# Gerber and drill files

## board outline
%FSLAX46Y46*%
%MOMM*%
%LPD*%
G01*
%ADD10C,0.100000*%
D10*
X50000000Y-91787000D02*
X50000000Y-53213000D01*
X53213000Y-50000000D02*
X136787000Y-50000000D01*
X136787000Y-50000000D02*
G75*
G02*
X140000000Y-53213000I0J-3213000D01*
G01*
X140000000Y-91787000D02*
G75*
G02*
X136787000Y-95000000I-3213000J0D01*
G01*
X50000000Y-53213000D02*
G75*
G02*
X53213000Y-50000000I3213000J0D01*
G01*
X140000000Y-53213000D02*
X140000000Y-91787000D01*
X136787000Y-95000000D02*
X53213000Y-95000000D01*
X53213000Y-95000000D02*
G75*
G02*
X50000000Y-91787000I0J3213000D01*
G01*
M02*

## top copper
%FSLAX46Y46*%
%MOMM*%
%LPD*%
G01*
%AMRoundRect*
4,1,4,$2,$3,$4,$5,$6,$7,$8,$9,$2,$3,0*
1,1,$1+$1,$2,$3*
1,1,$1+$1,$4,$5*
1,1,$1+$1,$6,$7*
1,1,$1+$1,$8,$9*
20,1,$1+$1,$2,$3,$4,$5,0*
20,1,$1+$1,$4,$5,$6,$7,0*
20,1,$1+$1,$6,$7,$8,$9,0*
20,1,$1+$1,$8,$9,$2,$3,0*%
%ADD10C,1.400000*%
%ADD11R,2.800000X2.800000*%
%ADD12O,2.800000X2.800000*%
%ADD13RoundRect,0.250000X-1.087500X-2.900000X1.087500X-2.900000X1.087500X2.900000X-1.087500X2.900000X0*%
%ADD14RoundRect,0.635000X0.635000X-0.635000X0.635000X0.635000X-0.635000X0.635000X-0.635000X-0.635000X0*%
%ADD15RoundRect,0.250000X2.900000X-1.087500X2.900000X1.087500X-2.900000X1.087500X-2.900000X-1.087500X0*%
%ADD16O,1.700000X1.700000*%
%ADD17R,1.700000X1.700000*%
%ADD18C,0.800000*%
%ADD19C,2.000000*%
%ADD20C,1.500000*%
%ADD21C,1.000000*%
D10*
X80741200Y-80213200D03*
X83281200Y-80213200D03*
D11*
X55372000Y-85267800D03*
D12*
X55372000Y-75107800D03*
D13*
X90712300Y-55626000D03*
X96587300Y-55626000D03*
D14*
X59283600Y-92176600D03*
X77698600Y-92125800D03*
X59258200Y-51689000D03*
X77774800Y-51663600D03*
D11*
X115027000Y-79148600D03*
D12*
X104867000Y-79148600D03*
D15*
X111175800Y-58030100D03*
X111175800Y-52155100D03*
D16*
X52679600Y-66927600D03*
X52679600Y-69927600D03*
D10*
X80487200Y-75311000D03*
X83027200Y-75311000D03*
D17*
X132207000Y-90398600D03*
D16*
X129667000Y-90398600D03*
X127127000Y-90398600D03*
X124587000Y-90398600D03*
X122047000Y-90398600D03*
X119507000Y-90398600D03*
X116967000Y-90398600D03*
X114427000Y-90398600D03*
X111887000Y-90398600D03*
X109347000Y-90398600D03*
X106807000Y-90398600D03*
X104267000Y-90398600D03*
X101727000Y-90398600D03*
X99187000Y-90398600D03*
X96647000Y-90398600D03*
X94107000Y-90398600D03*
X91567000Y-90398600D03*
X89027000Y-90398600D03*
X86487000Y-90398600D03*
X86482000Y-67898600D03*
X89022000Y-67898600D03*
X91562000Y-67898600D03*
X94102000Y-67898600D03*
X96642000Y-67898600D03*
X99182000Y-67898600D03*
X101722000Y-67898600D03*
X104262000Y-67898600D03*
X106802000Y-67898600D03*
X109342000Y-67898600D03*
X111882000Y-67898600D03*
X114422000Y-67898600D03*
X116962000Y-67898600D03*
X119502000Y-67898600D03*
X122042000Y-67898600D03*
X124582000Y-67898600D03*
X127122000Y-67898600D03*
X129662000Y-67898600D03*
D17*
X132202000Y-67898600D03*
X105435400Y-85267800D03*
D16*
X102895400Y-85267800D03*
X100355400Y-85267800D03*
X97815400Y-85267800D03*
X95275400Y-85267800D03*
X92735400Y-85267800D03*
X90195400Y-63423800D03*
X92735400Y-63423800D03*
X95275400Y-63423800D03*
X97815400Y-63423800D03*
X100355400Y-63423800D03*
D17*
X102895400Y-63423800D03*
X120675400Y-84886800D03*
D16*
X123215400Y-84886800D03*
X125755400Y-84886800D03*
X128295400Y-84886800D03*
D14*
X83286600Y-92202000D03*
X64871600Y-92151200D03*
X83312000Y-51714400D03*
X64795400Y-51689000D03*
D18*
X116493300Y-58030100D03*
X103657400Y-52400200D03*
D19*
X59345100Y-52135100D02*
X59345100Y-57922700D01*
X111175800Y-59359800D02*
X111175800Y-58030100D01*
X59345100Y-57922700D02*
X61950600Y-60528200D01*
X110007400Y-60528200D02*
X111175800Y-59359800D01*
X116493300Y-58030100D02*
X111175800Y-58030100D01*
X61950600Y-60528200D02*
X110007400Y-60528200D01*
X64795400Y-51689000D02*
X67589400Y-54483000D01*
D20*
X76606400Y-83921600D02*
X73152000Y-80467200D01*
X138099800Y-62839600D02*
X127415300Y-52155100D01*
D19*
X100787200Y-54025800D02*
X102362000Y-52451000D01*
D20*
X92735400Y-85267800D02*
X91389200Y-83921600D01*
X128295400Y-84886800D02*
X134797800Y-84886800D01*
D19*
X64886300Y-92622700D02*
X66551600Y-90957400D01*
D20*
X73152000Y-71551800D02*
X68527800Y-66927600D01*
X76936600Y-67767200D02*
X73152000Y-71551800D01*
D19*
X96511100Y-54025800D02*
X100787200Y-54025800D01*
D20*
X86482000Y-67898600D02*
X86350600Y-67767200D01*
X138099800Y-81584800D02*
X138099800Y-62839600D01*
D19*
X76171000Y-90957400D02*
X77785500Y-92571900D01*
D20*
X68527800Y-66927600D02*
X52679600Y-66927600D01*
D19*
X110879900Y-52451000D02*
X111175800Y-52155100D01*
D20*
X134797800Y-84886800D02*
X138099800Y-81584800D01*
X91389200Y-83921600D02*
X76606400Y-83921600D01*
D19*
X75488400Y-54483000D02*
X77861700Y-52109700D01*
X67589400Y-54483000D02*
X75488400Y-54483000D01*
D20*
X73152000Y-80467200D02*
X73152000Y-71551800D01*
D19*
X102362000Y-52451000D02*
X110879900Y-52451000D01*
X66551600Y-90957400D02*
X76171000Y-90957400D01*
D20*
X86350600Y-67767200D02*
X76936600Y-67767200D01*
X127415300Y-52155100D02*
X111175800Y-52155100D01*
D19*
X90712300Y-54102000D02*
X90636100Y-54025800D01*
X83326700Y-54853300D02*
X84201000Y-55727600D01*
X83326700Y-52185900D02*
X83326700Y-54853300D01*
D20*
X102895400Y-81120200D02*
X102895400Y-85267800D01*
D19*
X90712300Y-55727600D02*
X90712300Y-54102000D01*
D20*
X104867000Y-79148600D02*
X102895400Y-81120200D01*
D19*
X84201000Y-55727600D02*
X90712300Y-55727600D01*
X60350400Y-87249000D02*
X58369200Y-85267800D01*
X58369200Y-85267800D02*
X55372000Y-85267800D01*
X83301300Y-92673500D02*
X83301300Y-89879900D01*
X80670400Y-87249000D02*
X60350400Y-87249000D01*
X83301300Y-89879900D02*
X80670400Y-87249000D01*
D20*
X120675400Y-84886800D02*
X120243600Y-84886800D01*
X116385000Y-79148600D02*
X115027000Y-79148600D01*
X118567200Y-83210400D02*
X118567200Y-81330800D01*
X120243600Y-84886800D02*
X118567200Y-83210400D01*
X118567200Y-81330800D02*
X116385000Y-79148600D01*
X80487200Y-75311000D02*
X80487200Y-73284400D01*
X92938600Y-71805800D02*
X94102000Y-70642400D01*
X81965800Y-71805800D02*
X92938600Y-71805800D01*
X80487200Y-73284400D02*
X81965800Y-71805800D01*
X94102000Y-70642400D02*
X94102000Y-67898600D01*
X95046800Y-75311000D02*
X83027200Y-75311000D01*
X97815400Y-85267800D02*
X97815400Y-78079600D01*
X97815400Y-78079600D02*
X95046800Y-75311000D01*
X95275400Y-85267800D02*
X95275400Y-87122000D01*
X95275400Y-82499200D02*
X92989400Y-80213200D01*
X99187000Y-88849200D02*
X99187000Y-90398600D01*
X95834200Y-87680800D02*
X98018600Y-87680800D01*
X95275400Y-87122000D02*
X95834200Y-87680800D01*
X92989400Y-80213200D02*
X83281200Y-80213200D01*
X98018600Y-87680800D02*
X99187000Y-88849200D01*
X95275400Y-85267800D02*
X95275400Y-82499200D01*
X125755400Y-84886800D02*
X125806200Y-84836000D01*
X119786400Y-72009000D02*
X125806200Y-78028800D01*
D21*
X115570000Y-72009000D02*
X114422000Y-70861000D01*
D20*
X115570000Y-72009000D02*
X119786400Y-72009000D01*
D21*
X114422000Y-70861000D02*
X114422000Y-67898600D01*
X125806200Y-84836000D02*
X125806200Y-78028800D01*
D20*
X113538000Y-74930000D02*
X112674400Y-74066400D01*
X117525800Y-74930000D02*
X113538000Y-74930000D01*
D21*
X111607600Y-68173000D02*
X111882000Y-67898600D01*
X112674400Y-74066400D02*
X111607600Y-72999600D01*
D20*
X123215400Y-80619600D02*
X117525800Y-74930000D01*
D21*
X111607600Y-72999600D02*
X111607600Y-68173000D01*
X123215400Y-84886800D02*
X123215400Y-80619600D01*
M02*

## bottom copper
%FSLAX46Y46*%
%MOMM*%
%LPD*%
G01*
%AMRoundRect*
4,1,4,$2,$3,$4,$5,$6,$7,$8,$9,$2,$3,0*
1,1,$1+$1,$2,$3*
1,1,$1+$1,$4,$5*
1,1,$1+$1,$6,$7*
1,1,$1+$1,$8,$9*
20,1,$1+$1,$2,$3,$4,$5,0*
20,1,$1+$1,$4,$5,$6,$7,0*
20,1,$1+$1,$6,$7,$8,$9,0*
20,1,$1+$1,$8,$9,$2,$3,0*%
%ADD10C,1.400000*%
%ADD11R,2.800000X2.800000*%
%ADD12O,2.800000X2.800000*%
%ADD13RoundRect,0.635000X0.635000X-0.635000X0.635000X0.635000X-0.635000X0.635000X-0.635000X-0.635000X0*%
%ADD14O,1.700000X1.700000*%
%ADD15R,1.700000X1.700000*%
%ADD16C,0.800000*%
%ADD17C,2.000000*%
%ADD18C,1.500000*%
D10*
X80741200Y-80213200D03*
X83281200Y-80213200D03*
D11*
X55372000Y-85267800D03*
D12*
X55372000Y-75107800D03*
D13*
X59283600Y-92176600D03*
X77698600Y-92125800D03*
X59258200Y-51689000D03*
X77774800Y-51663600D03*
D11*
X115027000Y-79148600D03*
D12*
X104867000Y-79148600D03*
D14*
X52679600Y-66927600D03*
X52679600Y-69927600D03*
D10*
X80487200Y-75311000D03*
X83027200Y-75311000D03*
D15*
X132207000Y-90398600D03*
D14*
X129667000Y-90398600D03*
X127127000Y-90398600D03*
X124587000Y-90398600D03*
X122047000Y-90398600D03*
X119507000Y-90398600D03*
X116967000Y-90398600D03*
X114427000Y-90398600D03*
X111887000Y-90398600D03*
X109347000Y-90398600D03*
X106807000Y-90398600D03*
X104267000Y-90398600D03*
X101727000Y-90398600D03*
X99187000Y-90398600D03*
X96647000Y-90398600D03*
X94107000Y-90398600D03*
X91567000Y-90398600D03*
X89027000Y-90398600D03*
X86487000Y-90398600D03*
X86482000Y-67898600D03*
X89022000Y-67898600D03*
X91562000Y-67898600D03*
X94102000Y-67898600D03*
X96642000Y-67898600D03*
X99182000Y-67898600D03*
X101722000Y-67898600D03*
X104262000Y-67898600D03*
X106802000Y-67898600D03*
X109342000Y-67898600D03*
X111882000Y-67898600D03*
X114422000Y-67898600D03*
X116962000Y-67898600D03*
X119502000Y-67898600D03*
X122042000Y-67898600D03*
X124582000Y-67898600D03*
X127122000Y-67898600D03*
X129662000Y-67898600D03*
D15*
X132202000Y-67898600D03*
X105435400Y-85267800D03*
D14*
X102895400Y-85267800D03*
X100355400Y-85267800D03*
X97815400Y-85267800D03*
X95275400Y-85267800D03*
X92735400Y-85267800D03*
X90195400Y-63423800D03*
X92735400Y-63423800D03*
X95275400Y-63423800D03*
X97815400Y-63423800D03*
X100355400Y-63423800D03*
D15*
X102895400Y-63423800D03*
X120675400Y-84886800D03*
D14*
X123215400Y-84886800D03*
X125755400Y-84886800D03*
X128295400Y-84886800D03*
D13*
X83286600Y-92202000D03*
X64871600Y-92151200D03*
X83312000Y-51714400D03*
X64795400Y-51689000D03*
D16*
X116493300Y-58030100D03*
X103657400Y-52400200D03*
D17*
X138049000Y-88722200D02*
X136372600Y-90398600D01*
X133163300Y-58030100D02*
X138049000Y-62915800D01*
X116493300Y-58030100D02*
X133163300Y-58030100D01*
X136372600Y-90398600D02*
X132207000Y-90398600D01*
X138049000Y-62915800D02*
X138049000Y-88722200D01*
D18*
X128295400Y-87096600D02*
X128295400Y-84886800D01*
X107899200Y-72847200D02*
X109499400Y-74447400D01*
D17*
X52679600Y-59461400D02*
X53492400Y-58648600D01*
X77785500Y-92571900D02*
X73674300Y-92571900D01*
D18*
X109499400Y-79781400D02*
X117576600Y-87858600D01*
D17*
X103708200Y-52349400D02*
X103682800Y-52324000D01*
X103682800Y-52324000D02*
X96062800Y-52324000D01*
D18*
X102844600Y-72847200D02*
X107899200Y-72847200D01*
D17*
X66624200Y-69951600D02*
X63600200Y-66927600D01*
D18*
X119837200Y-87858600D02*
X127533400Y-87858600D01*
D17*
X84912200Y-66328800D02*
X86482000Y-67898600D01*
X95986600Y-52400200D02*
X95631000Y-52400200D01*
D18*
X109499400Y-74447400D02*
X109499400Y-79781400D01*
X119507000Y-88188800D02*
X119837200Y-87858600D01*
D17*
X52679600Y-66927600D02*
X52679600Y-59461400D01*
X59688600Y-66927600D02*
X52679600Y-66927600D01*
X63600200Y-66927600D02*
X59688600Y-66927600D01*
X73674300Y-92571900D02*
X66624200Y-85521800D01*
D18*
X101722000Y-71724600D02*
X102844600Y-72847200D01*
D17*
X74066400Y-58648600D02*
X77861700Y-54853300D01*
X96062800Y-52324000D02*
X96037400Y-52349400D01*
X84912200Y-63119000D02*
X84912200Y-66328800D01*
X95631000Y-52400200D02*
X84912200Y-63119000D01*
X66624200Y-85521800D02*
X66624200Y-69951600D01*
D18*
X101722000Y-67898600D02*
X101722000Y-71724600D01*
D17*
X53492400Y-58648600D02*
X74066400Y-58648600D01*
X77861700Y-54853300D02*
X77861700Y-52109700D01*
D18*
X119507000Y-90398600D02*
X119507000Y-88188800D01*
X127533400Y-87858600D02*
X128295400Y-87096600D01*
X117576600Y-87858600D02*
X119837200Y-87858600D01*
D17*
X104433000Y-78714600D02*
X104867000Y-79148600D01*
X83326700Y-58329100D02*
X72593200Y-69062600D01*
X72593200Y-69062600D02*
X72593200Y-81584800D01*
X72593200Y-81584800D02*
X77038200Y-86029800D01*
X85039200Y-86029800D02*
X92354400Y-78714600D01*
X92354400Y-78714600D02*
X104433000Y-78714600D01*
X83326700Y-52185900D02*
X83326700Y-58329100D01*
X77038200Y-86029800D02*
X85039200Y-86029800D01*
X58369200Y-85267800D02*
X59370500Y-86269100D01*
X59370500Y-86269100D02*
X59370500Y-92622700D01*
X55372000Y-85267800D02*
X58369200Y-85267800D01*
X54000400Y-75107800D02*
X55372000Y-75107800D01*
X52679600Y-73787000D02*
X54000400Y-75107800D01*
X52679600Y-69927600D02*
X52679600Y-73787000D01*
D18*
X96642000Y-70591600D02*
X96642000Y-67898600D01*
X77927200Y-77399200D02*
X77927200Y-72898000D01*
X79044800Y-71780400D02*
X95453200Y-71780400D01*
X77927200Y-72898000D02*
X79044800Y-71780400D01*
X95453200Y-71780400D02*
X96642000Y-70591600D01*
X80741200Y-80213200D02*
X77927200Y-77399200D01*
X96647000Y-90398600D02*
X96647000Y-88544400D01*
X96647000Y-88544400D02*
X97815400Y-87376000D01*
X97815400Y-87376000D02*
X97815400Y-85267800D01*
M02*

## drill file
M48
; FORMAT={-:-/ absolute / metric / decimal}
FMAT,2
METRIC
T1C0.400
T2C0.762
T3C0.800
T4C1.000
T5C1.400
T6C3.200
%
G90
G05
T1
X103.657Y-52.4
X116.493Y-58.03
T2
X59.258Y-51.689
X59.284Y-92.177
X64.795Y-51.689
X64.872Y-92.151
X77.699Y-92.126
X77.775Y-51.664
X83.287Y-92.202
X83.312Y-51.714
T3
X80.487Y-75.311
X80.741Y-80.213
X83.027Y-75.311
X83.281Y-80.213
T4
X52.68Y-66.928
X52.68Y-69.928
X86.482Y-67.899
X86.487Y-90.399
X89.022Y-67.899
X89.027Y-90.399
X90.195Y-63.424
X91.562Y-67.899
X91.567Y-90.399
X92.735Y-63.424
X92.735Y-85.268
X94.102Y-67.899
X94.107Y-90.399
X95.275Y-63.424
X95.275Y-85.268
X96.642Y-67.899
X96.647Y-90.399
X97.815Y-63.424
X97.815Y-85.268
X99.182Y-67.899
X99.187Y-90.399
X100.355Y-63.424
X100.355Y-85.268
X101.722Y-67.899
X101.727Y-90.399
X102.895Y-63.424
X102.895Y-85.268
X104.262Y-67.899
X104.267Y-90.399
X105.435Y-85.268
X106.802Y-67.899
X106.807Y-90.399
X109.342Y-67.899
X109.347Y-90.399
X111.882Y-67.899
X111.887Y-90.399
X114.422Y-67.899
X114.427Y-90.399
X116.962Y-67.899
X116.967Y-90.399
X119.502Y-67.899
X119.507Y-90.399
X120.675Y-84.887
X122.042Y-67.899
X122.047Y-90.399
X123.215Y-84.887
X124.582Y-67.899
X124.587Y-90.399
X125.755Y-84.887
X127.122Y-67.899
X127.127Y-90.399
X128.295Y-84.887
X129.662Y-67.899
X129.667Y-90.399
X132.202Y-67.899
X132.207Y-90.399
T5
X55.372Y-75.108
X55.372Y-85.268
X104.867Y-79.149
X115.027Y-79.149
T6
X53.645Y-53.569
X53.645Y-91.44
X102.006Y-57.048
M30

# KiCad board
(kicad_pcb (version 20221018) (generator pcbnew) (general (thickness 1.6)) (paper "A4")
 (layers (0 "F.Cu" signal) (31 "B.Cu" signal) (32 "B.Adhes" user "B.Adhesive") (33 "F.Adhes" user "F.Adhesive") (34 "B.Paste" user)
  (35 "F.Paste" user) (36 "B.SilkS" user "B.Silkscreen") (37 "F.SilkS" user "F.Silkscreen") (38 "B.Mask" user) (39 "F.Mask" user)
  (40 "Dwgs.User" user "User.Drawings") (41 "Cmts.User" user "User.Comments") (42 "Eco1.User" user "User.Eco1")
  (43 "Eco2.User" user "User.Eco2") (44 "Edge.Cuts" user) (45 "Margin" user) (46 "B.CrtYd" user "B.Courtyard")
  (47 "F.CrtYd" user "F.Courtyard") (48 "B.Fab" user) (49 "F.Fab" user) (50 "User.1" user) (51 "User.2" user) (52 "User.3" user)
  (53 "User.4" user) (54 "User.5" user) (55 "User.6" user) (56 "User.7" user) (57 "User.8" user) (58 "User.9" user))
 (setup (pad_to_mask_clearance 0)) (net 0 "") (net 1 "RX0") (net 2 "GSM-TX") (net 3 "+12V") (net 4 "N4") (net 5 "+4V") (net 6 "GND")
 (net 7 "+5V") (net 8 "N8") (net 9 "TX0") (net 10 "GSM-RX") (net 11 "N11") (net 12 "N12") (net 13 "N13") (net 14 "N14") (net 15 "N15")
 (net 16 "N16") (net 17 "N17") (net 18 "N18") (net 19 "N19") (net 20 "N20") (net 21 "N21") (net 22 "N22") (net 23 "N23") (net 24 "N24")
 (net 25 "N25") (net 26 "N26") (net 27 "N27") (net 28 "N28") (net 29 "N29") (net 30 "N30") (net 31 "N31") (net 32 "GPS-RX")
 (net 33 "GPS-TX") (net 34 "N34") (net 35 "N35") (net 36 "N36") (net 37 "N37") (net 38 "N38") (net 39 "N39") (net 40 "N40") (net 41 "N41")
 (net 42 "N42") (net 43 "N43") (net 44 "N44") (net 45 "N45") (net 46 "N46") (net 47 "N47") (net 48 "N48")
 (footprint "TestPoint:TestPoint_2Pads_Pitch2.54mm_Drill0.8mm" (layer "F.Cu") (at 80.7412 80.2132)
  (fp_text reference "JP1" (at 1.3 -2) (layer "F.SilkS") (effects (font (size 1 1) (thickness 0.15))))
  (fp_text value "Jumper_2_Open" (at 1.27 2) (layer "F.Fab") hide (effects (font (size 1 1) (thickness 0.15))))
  (pad "1" thru_hole circle (at 0 0) (size 1.4 1.4) (drill 0.8) (layers "*.Cu" "*.Mask") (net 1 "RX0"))
  (pad "2" thru_hole circle (at 2.54 0) (size 1.4 1.4) (drill 0.8) (layers "*.Cu" "*.Mask") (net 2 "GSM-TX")))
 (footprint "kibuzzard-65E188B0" (layer "F.Cu") (at 52.2224 64.2874)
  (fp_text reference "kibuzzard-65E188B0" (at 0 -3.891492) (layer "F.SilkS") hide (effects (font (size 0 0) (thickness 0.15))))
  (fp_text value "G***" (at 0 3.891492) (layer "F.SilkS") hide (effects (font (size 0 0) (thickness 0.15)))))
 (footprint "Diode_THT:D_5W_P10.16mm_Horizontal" (layer "F.Cu") (at 55.372 85.2678 90)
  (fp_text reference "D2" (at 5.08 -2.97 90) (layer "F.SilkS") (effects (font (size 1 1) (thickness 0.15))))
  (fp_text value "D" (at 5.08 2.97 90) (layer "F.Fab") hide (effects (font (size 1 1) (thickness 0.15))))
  (pad "1" thru_hole rect (at 0 0 90) (size 2.8 2.8) (drill 1.4) (layers "*.Cu" "*.Mask") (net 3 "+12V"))
  (pad "2" thru_hole oval (at 10.16 0 90) (size 2.8 2.8) (drill 1.4) (layers "*.Cu" "*.Mask") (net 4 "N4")))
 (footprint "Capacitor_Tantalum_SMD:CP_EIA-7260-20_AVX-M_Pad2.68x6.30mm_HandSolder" (layer "F.Cu") (at 93.6498 55.626)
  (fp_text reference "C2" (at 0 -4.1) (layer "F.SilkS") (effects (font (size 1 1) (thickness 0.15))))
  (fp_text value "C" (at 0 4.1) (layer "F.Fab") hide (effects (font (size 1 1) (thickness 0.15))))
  (pad "1" smd roundrect (at -2.9375 0) (size 2.675 6.3) (layers "F.Cu" "F.Paste" "F.Mask") (roundrect_rratio 0.093458) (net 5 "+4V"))
  (pad "2" smd roundrect (at 2.9375 0) (size 2.675 6.3) (layers "F.Cu" "F.Paste" "F.Mask") (roundrect_rratio 0.093458) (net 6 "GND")))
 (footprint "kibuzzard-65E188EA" (layer "F.Cu") (at 52.1716 72.5424)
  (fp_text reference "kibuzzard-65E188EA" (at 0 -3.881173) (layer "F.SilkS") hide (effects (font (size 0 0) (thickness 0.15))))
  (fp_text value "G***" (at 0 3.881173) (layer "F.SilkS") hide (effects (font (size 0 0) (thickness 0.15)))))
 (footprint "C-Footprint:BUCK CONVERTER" (layer "F.Cu") (at 57.9882 93.4212 90)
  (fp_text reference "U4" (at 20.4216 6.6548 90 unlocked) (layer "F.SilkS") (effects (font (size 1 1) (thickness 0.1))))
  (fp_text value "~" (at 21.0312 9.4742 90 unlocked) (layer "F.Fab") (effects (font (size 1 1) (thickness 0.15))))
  (pad "1" thru_hole roundrect (at 1.2446 1.2954 90) (size 2.54 2.54) (drill 0.762) (layers "*.Cu" "*.Mask") (roundrect_rratio 0.25)
   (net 3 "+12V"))
  (pad "2" thru_hole roundrect (at 1.2954 19.7104 90) (size 2.54 2.54) (drill 0.762) (layers "*.Cu" "*.Mask") (roundrect_rratio 0.25)
   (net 6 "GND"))
  (pad "3" thru_hole roundrect (at 41.7322 1.27 90) (size 2.54 2.54) (drill 0.762) (layers "*.Cu" "*.Mask") (roundrect_rratio 0.25)
   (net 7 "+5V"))
  (pad "4" thru_hole roundrect (at 41.7576 19.7866 90) (size 2.54 2.54) (drill 0.762) (layers "*.Cu" "*.Mask") (roundrect_rratio 0.25)
   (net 6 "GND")))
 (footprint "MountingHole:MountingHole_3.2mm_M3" (layer "F.Cu") (at 102.0064 57.0484)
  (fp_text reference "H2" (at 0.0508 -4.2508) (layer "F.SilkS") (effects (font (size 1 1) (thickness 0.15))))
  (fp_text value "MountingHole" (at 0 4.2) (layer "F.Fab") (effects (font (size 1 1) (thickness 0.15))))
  (pad "" np_thru_hole circle (at 0 0) (size 3.2 3.2) (drill 3.2) (layers "*.Cu" "*.Mask")))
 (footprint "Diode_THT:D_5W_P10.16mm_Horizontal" (layer "F.Cu") (at 115.027 79.1486 180)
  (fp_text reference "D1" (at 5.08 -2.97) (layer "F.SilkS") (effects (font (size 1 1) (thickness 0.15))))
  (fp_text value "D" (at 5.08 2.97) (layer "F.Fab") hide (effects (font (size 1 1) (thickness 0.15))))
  (pad "1" thru_hole rect (at 0 0 180) (size 2.8 2.8) (drill 1.4) (layers "*.Cu" "*.Mask") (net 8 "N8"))
  (pad "2" thru_hole oval (at 10.16 0 180) (size 2.8 2.8) (drill 1.4) (layers "*.Cu" "*.Mask") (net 5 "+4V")))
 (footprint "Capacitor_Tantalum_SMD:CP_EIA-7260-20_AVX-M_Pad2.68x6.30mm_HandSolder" (layer "F.Cu") (at 111.1758 55.0926 90)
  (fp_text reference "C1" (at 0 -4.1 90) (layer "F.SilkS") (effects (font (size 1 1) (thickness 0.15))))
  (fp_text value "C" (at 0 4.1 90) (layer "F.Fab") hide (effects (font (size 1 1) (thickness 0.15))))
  (pad "1" smd roundrect (at -2.9375 0 90) (size 2.675 6.3) (layers "F.Cu" "F.Paste" "F.Mask") (roundrect_rratio 0.093458) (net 7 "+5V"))
  (pad "2" smd roundrect (at 2.9375 0 90) (size 2.675 6.3) (layers "F.Cu" "F.Paste" "F.Mask") (roundrect_rratio 0.093458) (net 6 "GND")))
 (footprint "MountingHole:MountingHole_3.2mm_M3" (layer "F.Cu") (at 53.6448 53.5686)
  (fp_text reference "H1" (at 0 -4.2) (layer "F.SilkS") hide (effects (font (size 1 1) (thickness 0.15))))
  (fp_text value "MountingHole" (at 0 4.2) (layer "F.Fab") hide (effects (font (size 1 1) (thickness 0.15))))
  (pad "" np_thru_hole circle (at 0 0) (size 3.2 3.2) (drill 3.2) (layers "*.Cu" "*.Mask")))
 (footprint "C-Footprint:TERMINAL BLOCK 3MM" (layer "F.Cu") (at 52.6796 66.9276 -90)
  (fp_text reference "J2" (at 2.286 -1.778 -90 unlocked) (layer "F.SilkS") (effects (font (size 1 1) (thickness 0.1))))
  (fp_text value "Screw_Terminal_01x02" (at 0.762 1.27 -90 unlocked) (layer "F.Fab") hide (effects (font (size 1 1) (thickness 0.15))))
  (pad "1" thru_hole oval (at 0 0 270) (size 1.7 1.7) (drill 1) (layers "*.Cu" "*.Mask") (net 6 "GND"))
  (pad "2" thru_hole oval (at 3 0 270) (size 1.7 1.7) (drill 1) (layers "*.Cu" "*.Mask") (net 4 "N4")))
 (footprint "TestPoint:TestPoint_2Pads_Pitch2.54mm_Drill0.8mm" (layer "F.Cu") (at 80.4872 75.311)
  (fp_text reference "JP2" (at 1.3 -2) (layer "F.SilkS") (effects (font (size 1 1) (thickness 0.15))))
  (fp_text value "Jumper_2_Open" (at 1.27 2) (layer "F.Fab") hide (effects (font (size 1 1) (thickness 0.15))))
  (pad "1" thru_hole circle (at 0 0) (size 1.4 1.4) (drill 0.8) (layers "*.Cu" "*.Mask") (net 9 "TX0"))
  (pad "2" thru_hole circle (at 2.54 0) (size 1.4 1.4) (drill 0.8) (layers "*.Cu" "*.Mask") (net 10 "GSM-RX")))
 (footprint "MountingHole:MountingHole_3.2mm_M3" (layer "F.Cu") (at 53.6448 91.44)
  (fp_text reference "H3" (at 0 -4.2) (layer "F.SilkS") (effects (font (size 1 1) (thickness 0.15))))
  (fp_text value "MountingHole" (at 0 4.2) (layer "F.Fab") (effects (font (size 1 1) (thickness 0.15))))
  (pad "" np_thru_hole circle (at 0 0) (size 3.2 3.2) (drill 3.2) (layers "*.Cu" "*.Mask")))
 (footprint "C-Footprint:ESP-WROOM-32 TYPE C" (layer "F.Cu") (at 110.157 67.8986 -90)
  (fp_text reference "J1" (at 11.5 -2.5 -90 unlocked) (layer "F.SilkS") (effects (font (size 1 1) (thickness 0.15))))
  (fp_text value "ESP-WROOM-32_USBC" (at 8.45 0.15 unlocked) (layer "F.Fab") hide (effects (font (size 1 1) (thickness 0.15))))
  (pad "1" thru_hole rect (at 22.5 -22.05 270) (size 1.7 1.7) (drill 1) (layers "*.Cu" "*.Mask") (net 7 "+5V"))
  (pad "2" thru_hole oval (at 22.5 -19.51 270) (size 1.7 1.7) (drill 1) (layers "*.Cu" "*.Mask") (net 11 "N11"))
  (pad "3" thru_hole oval (at 22.5 -16.97 270) (size 1.7 1.7) (drill 1) (layers "*.Cu" "*.Mask") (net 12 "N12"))
  (pad "4" thru_hole oval (at 22.5 -14.43 270) (size 1.7 1.7) (drill 1) (layers "*.Cu" "*.Mask") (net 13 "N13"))
  (pad "5" thru_hole oval (at 22.5 -11.89 270) (size 1.7 1.7) (drill 1) (layers "*.Cu" "*.Mask") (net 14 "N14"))
  (pad "6" thru_hole oval (at 22.5 -9.35 270) (size 1.7 1.7) (drill 1) (layers "*.Cu" "*.Mask") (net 6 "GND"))
  (pad "7" thru_hole oval (at 22.5 -6.81 270) (size 1.7 1.7) (drill 1) (layers "*.Cu" "*.Mask") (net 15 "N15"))
  (pad "8" thru_hole oval (at 22.5 -4.27 270) (size 1.7 1.7) (drill 1) (layers "*.Cu" "*.Mask") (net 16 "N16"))
  (pad "9" thru_hole oval (at 22.5 -1.73 270) (size 1.7 1.7) (drill 1) (layers "*.Cu" "*.Mask") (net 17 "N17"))
  (pad "10" thru_hole oval (at 22.5 0.81 270) (size 1.7 1.7) (drill 1) (layers "*.Cu" "*.Mask") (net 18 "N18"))
  (pad "11" thru_hole oval (at 22.5 3.35 270) (size 1.7 1.7) (drill 1) (layers "*.Cu" "*.Mask") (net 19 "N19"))
  (pad "12" thru_hole oval (at 22.5 5.89 270) (size 1.7 1.7) (drill 1) (layers "*.Cu" "*.Mask") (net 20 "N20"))
  (pad "13" thru_hole oval (at 22.5 8.43 270) (size 1.7 1.7) (drill 1) (layers "*.Cu" "*.Mask") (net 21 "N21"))
  (pad "14" thru_hole oval (at 22.5 10.97 270) (size 1.7 1.7) (drill 1) (layers "*.Cu" "*.Mask") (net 2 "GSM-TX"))
  (pad "15" thru_hole oval (at 22.5 13.51 270) (size 1.7 1.7) (drill 1) (layers "*.Cu" "*.Mask") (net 10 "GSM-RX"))
  (pad "16" thru_hole oval (at 22.5 16.05 270) (size 1.7 1.7) (drill 1) (layers "*.Cu" "*.Mask") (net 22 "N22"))
  (pad "17" thru_hole oval (at 22.5 18.59 270) (size 1.7 1.7) (drill 1) (layers "*.Cu" "*.Mask") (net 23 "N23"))
  (pad "18" thru_hole oval (at 22.5 21.13 270) (size 1.7 1.7) (drill 1) (layers "*.Cu" "*.Mask") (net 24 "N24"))
  (pad "19" thru_hole oval (at 22.5 23.67 270) (size 1.7 1.7) (drill 1) (layers "*.Cu" "*.Mask") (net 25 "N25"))
  (pad "20" thru_hole oval (at 0 23.675 270) (size 1.7 1.7) (drill 1) (layers "*.Cu" "*.Mask") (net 6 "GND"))
  (pad "21" thru_hole oval (at 0 21.135 270) (size 1.7 1.7) (drill 1) (layers "*.Cu" "*.Mask") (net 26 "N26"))
  (pad "22" thru_hole oval (at 0 18.595 270) (size 1.7 1.7) (drill 1) (layers "*.Cu" "*.Mask") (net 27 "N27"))
  (pad "23" thru_hole oval (at 0 16.055 270) (size 1.7 1.7) (drill 1) (layers "*.Cu" "*.Mask") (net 9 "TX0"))
  (pad "24" thru_hole oval (at 0 13.515 270) (size 1.7 1.7) (drill 1) (layers "*.Cu" "*.Mask") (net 1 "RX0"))
  (pad "25" thru_hole oval (at 0 10.975 270) (size 1.7 1.7) (drill 1) (layers "*.Cu" "*.Mask") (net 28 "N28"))
  (pad "26" thru_hole oval (at 0 8.435 270) (size 1.7 1.7) (drill 1) (layers "*.Cu" "*.Mask") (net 6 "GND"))
  (pad "27" thru_hole oval (at 0 5.895 270) (size 1.7 1.7) (drill 1) (layers "*.Cu" "*.Mask") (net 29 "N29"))
  (pad "28" thru_hole oval (at 0 3.355 270) (size 1.7 1.7) (drill 1) (layers "*.Cu" "*.Mask") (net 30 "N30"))
  (pad "29" thru_hole oval (at 0 0.815 270) (size 1.7 1.7) (drill 1) (layers "*.Cu" "*.Mask") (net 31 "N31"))
  (pad "30" thru_hole oval (at 0 -1.725 270) (size 1.7 1.7) (drill 1) (layers "*.Cu" "*.Mask") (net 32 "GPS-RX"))
  (pad "31" thru_hole oval (at 0 -4.265 270) (size 1.7 1.7) (drill 1) (layers "*.Cu" "*.Mask") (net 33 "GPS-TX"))
  (pad "32" thru_hole oval (at 0 -6.805 270) (size 1.7 1.7) (drill 1) (layers "*.Cu" "*.Mask") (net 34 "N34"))
  (pad "33" thru_hole oval (at 0 -9.345 270) (size 1.7 1.7) (drill 1) (layers "*.Cu" "*.Mask") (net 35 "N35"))
  (pad "34" thru_hole oval (at 0 -11.885 270) (size 1.7 1.7) (drill 1) (layers "*.Cu" "*.Mask") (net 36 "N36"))
  (pad "35" thru_hole oval (at 0 -14.425 270) (size 1.7 1.7) (drill 1) (layers "*.Cu" "*.Mask") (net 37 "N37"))
  (pad "36" thru_hole oval (at 0 -16.965 270) (size 1.7 1.7) (drill 1) (layers "*.Cu" "*.Mask") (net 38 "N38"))
  (pad "37" thru_hole oval (at 0 -19.505 270) (size 1.7 1.7) (drill 1) (layers "*.Cu" "*.Mask") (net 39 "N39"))
  (pad "38" thru_hole rect (at 0 -22.045 270) (size 1.7 1.7) (drill 1) (layers "*.Cu" "*.Mask") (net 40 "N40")))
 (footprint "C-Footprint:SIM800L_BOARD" (layer "B.Cu") (at 110.0074 87.2998 90)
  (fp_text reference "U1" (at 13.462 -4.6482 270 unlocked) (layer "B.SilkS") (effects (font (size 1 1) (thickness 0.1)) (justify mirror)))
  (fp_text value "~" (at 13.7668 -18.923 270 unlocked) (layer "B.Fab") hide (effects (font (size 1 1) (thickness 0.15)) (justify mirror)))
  (pad "1" thru_hole rect (at 2.032 -4.572 90) (size 1.7 1.7) (drill 1) (layers "*.Cu" "*.Mask") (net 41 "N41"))
  (pad "2" thru_hole oval (at 2.032 -7.112 90) (size 1.7 1.7) (drill 1) (layers "*.Cu" "*.Mask") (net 5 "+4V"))
  (pad "3" thru_hole oval (at 2.032 -9.652 90) (size 1.7 1.7) (drill 1) (layers "*.Cu" "*.Mask") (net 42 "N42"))
  (pad "4" thru_hole oval (at 2.032 -12.192 90) (size 1.7 1.7) (drill 1) (layers "*.Cu" "*.Mask") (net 10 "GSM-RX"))
  (pad "5" thru_hole oval (at 2.032 -14.732 90) (size 1.7 1.7) (drill 1) (layers "*.Cu" "*.Mask") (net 2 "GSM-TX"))
  (pad "6" thru_hole oval (at 2.032 -17.272 90) (size 1.7 1.7) (drill 1) (layers "*.Cu" "*.Mask") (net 6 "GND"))
  (pad "7" thru_hole oval (at 23.876 -19.812 90) (size 1.7 1.7) (drill 1) (layers "*.Cu" "*.Mask") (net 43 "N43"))
  (pad "8" thru_hole oval (at 23.876 -17.272 90) (size 1.7 1.7) (drill 1) (layers "*.Cu" "*.Mask") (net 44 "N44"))
  (pad "9" thru_hole oval (at 23.876 -14.732 90) (size 1.7 1.7) (drill 1) (layers "*.Cu" "*.Mask") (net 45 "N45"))
  (pad "10" thru_hole oval (at 23.876 -12.192 90) (size 1.7 1.7) (drill 1) (layers "*.Cu" "*.Mask") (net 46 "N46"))
  (pad "11" thru_hole oval (at 23.876 -9.652 90) (size 1.7 1.7) (drill 1) (layers "*.Cu" "*.Mask") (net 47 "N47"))
  (pad "12" thru_hole rect (at 23.876 -7.112 90) (size 1.7 1.7) (drill 1) (layers "*.Cu" "*.Mask") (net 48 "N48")))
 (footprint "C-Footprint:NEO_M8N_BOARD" (layer "B.Cu") (at 136.8044 87.0874 90)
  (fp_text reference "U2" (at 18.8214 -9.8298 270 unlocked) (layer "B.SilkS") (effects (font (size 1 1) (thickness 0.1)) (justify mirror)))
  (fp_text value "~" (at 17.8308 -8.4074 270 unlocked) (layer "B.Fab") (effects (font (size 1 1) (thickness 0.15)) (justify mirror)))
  (pad "1" thru_hole rect (at 2.2006 -16.129 270) (size 1.7 1.7) (drill 1) (layers "*.Cu" "*.Mask") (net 8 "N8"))
  (pad "2" thru_hole oval (at 2.2006 -13.589 270) (size 1.7 1.7) (drill 1) (layers "*.Cu" "*.Mask") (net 32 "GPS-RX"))
  (pad "3" thru_hole oval (at 2.2006 -11.049 270) (size 1.7 1.7) (drill 1) (layers "*.Cu" "*.Mask") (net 33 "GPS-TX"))
  (pad "4" thru_hole oval (at 2.2006 -8.509 270) (size 1.7 1.7) (drill 1) (layers "*.Cu" "*.Mask") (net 6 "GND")))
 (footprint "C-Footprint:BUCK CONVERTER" (layer "B.Cu") (at 84.582 93.4466 90)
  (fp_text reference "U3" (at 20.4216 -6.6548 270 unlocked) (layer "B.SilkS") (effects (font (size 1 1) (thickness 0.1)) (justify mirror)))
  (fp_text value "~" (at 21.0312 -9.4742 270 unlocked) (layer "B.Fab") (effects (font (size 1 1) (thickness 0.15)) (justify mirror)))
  (pad "1" thru_hole roundrect (at 1.2446 -1.2954 90) (size 2.54 2.54) (drill 0.762) (layers "*.Cu" "*.Mask") (roundrect_rratio 0.25)
   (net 3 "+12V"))
  (pad "2" thru_hole roundrect (at 1.2954 -19.7104 90) (size 2.54 2.54) (drill 0.762) (layers "*.Cu" "*.Mask") (roundrect_rratio 0.25)
   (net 6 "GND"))
  (pad "3" thru_hole roundrect (at 41.7322 -1.27 90) (size 2.54 2.54) (drill 0.762) (layers "*.Cu" "*.Mask") (roundrect_rratio 0.25)
   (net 5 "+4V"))
  (pad "4" thru_hole roundrect (at 41.7576 -19.7866 90) (size 2.54 2.54) (drill 0.762) (layers "*.Cu" "*.Mask") (roundrect_rratio 0.25)
   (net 6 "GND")))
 (gr_line (start 50 91.787) (end 50 53.213) (stroke (width 0.1) (type default)) (layer "Edge.Cuts"))
 (gr_line (start 53.213 50) (end 136.787 50) (stroke (width 0.1) (type default)) (layer "Edge.Cuts"))
 (gr_arc (start 136.787 50) (mid 139.058934 50.941066) (end 140 53.213) (stroke (width 0.1) (type default)) (layer "Edge.Cuts"))
 (gr_arc (start 140 91.787) (mid 139.058934 94.058934) (end 136.787 95) (stroke (width 0.1) (type default)) (layer "Edge.Cuts"))
 (gr_arc (start 50 53.213) (mid 50.941066 50.941066) (end 53.213 50) (stroke (width 0.1) (type default)) (layer "Edge.Cuts"))
 (gr_line (start 140 53.213) (end 140 91.787) (stroke (width 0.1) (type default)) (layer "Edge.Cuts"))
 (gr_line (start 136.787 95) (end 53.213 95) (stroke (width 0.1) (type default)) (layer "Edge.Cuts"))
 (gr_arc (start 53.213 95) (mid 50.941066 94.058934) (end 50 91.787) (stroke (width 0.1) (type default)) (layer "Edge.Cuts"))
 (segment (start 59.3451 52.1351) (end 59.3451 57.9227) (width 2) (layer "F.Cu") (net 7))
 (segment (start 111.1758 59.3598) (end 111.1758 58.0301) (width 2) (layer "F.Cu") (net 7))
 (segment (start 59.3451 57.9227) (end 61.9506 60.5282) (width 2) (layer "F.Cu") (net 7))
 (segment (start 110.0074 60.5282) (end 111.1758 59.3598) (width 2) (layer "F.Cu") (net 7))
 (segment (start 116.4933 58.0301) (end 111.1758 58.0301) (width 2) (layer "F.Cu") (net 7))
 (segment (start 61.9506 60.5282) (end 110.0074 60.5282) (width 2) (layer "F.Cu") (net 7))
 (via (at 116.4933 58.0301) (size 0.8) (drill 0.4) (layers "F.Cu" "B.Cu") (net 7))
 (segment (start 138.049 88.7222) (end 136.3726 90.3986) (width 2) (layer "B.Cu") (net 7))
 (segment (start 133.1633 58.0301) (end 138.049 62.9158) (width 2) (layer "B.Cu") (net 7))
 (segment (start 116.4933 58.0301) (end 133.1633 58.0301) (width 2) (layer "B.Cu") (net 7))
 (segment (start 136.3726 90.3986) (end 132.207 90.3986) (width 2) (layer "B.Cu") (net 7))
 (segment (start 138.049 62.9158) (end 138.049 88.7222) (width 2) (layer "B.Cu") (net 7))
 (segment (start 64.7954 51.689) (end 67.5894 54.483) (width 2) (layer "F.Cu") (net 6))
 (segment (start 76.6064 83.9216) (end 73.152 80.4672) (width 1.5) (layer "F.Cu") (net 6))
 (segment (start 138.0998 62.8396) (end 127.4153 52.1551) (width 1.5) (layer "F.Cu") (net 6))
 (segment (start 100.7872 54.0258) (end 102.362 52.451) (width 2) (layer "F.Cu") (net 6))
 (segment (start 92.7354 85.2678) (end 91.3892 83.9216) (width 1.5) (layer "F.Cu") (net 6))
 (segment (start 128.2954 84.8868) (end 134.7978 84.8868) (width 1.5) (layer "F.Cu") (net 6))
 (segment (start 64.8863 92.6227) (end 66.5516 90.9574) (width 2) (layer "F.Cu") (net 6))
 (segment (start 73.152 71.5518) (end 68.5278 66.9276) (width 1.5) (layer "F.Cu") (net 6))
 (segment (start 76.9366 67.7672) (end 73.152 71.5518) (width 1.5) (layer "F.Cu") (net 6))
 (segment (start 96.5111 54.0258) (end 100.7872 54.0258) (width 2) (layer "F.Cu") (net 6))
 (segment (start 86.482 67.8986) (end 86.3506 67.7672) (width 1.5) (layer "F.Cu") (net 6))
 (segment (start 138.0998 81.5848) (end 138.0998 62.8396) (width 1.5) (layer "F.Cu") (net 6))
 (segment (start 76.171 90.9574) (end 77.7855 92.5719) (width 2) (layer "F.Cu") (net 6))
 (segment (start 68.5278 66.9276) (end 52.6796 66.9276) (width 1.5) (layer "F.Cu") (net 6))
 (segment (start 110.8799 52.451) (end 111.1758 52.1551) (width 2) (layer "F.Cu") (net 6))
 (segment (start 134.7978 84.8868) (end 138.0998 81.5848) (width 1.5) (layer "F.Cu") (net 6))
 (segment (start 91.3892 83.9216) (end 76.6064 83.9216) (width 1.5) (layer "F.Cu") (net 6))
 (segment (start 75.4884 54.483) (end 77.8617 52.1097) (width 2) (layer "F.Cu") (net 6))
 (segment (start 67.5894 54.483) (end 75.4884 54.483) (width 2) (layer "F.Cu") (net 6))
 (segment (start 73.152 80.4672) (end 73.152 71.5518) (width 1.5) (layer "F.Cu") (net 6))
 (segment (start 102.362 52.451) (end 110.8799 52.451) (width 2) (layer "F.Cu") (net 6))
 (segment (start 66.5516 90.9574) (end 76.171 90.9574) (width 2) (layer "F.Cu") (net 6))
 (segment (start 86.3506 67.7672) (end 76.9366 67.7672) (width 1.5) (layer "F.Cu") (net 6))
 (segment (start 127.4153 52.1551) (end 111.1758 52.1551) (width 1.5) (layer "F.Cu") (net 6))
 (via (at 103.6574 52.4002) (size 0.8) (drill 0.4) (layers "F.Cu" "B.Cu") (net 6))
 (segment (start 128.2954 87.0966) (end 128.2954 84.8868) (width 1.5) (layer "B.Cu") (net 6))
 (segment (start 107.8992 72.8472) (end 109.4994 74.4474) (width 1.5) (layer "B.Cu") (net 6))
 (segment (start 52.6796 59.4614) (end 53.4924 58.6486) (width 2) (layer "B.Cu") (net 6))
 (segment (start 77.7855 92.5719) (end 73.6743 92.5719) (width 2) (layer "B.Cu") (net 6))
 (segment (start 109.4994 79.7814) (end 117.5766 87.8586) (width 1.5) (layer "B.Cu") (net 6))
 (segment (start 103.7082 52.3494) (end 103.6828 52.324) (width 2) (layer "B.Cu") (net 6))
 (segment (start 103.6828 52.324) (end 96.0628 52.324) (width 2) (layer "B.Cu") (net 6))
 (segment (start 102.8446 72.8472) (end 107.8992 72.8472) (width 1.5) (layer "B.Cu") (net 6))
 (segment (start 66.6242 69.9516) (end 63.6002 66.9276) (width 2) (layer "B.Cu") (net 6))
 (segment (start 119.8372 87.8586) (end 127.5334 87.8586) (width 1.5) (layer "B.Cu") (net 6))
 (segment (start 84.9122 66.3288) (end 86.482 67.8986) (width 2) (layer "B.Cu") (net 6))
 (segment (start 95.9866 52.4002) (end 95.631 52.4002) (width 2) (layer "B.Cu") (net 6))
 (segment (start 109.4994 74.4474) (end 109.4994 79.7814) (width 1.5) (layer "B.Cu") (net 6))
 (segment (start 119.507 88.1888) (end 119.8372 87.8586) (width 1.5) (layer "B.Cu") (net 6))
 (segment (start 52.6796 66.9276) (end 52.6796 59.4614) (width 2) (layer "B.Cu") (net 6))
 (segment (start 59.6886 66.9276) (end 52.6796 66.9276) (width 2) (layer "B.Cu") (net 6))
 (segment (start 63.6002 66.9276) (end 59.6886 66.9276) (width 2) (layer "B.Cu") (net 6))
 (segment (start 73.6743 92.5719) (end 66.6242 85.5218) (width 2) (layer "B.Cu") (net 6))
 (segment (start 101.722 71.7246) (end 102.8446 72.8472) (width 1.5) (layer "B.Cu") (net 6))
 (segment (start 74.0664 58.6486) (end 77.8617 54.8533) (width 2) (layer "B.Cu") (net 6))
 (segment (start 96.0628 52.324) (end 96.0374 52.3494) (width 2) (layer "B.Cu") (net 6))
 (segment (start 84.9122 63.119) (end 84.9122 66.3288) (width 2) (layer "B.Cu") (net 6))
 (segment (start 95.631 52.4002) (end 84.9122 63.119) (width 2) (layer "B.Cu") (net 6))
 (segment (start 66.6242 85.5218) (end 66.6242 69.9516) (width 2) (layer "B.Cu") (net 6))
 (segment (start 101.722 67.8986) (end 101.722 71.7246) (width 1.5) (layer "B.Cu") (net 6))
 (segment (start 53.4924 58.6486) (end 74.0664 58.6486) (width 2) (layer "B.Cu") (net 6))
 (segment (start 77.8617 54.8533) (end 77.8617 52.1097) (width 2) (layer "B.Cu") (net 6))
 (segment (start 119.507 90.3986) (end 119.507 88.1888) (width 1.5) (layer "B.Cu") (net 6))
 (segment (start 127.5334 87.8586) (end 128.2954 87.0966) (width 1.5) (layer "B.Cu") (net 6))
 (segment (start 117.5766 87.8586) (end 119.8372 87.8586) (width 1.5) (layer "B.Cu") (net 6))
 (segment (start 90.7123 54.102) (end 90.6361 54.0258) (width 2) (layer "F.Cu") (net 5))
 (segment (start 83.3267 54.8533) (end 84.201 55.7276) (width 2) (layer "F.Cu") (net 5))
 (segment (start 83.3267 52.1859) (end 83.3267 54.8533) (width 2) (layer "F.Cu") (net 5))
 (segment (start 102.8954 81.1202) (end 102.8954 85.2678) (width 1.5) (layer "F.Cu") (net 5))
 (segment (start 90.7123 55.7276) (end 90.7123 54.102) (width 2) (layer "F.Cu") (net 5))
 (segment (start 104.867 79.1486) (end 102.8954 81.1202) (width 1.5) (layer "F.Cu") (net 5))
 (segment (start 84.201 55.7276) (end 90.7123 55.7276) (width 2) (layer "F.Cu") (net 5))
 (segment (start 104.433 78.7146) (end 104.867 79.1486) (width 2) (layer "B.Cu") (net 5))
 (segment (start 83.3267 58.3291) (end 72.5932 69.0626) (width 2) (layer "B.Cu") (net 5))
 (segment (start 72.5932 69.0626) (end 72.5932 81.5848) (width 2) (layer "B.Cu") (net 5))
 (segment (start 72.5932 81.5848) (end 77.0382 86.0298) (width 2) (layer "B.Cu") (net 5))
 (segment (start 85.0392 86.0298) (end 92.3544 78.7146) (width 2) (layer "B.Cu") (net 5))
 (segment (start 92.3544 78.7146) (end 104.433 78.7146) (width 2) (layer "B.Cu") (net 5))
 (segment (start 83.3267 52.1859) (end 83.3267 58.3291) (width 2) (layer "B.Cu") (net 5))
 (segment (start 77.0382 86.0298) (end 85.0392 86.0298) (width 2) (layer "B.Cu") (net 5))
 (segment (start 60.3504 87.249) (end 58.3692 85.2678) (width 2) (layer "F.Cu") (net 3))
 (segment (start 58.3692 85.2678) (end 55.372 85.2678) (width 2) (layer "F.Cu") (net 3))
 (segment (start 83.3013 92.6735) (end 83.3013 89.8799) (width 2) (layer "F.Cu") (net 3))
 (segment (start 80.6704 87.249) (end 60.3504 87.249) (width 2) (layer "F.Cu") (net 3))
 (segment (start 83.3013 89.8799) (end 80.6704 87.249) (width 2) (layer "F.Cu") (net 3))
 (segment (start 58.3692 85.2678) (end 59.3705 86.2691) (width 2) (layer "B.Cu") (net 3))
 (segment (start 59.3705 86.2691) (end 59.3705 92.6227) (width 2) (layer "B.Cu") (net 3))
 (segment (start 55.372 85.2678) (end 58.3692 85.2678) (width 2) (layer "B.Cu") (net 3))
 (segment (start 120.6754 84.8868) (end 120.2436 84.8868) (width 1.5) (layer "F.Cu") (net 8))
 (segment (start 116.385 79.1486) (end 115.027 79.1486) (width 1.5) (layer "F.Cu") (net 8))
 (segment (start 118.5672 83.2104) (end 118.5672 81.3308) (width 1.5) (layer "F.Cu") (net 8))
 (segment (start 120.2436 84.8868) (end 118.5672 83.2104) (width 1.5) (layer "F.Cu") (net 8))
 (segment (start 118.5672 81.3308) (end 116.385 79.1486) (width 1.5) (layer "F.Cu") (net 8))
 (segment (start 54.0004 75.1078) (end 55.372 75.1078) (width 2) (layer "B.Cu") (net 4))
 (segment (start 52.6796 73.787) (end 54.0004 75.1078) (width 2) (layer "B.Cu") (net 4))
 (segment (start 52.6796 69.9276) (end 52.6796 73.787) (width 2) (layer "B.Cu") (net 4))
 (segment (start 96.642 70.5916) (end 96.642 67.8986) (width 1.5) (layer "B.Cu") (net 1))
 (segment (start 77.9272 77.3992) (end 77.9272 72.898) (width 1.5) (layer "B.Cu") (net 1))
 (segment (start 79.0448 71.7804) (end 95.4532 71.7804) (width 1.5) (layer "B.Cu") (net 1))
 (segment (start 77.9272 72.898) (end 79.0448 71.7804) (width 1.5) (layer "B.Cu") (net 1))
 (segment (start 95.4532 71.7804) (end 96.642 70.5916) (width 1.5) (layer "B.Cu") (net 1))
 (segment (start 80.7412 80.2132) (end 77.9272 77.3992) (width 1.5) (layer "B.Cu") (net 1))
 (segment (start 80.4872 75.311) (end 80.4872 73.2844) (width 1.5) (layer "F.Cu") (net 9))
 (segment (start 92.9386 71.8058) (end 94.102 70.6424) (width 1.5) (layer "F.Cu") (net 9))
 (segment (start 81.9658 71.8058) (end 92.9386 71.8058) (width 1.5) (layer "F.Cu") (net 9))
 (segment (start 80.4872 73.2844) (end 81.9658 71.8058) (width 1.5) (layer "F.Cu") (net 9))
 (segment (start 94.102 70.6424) (end 94.102 67.8986) (width 1.5) (layer "F.Cu") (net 9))
 (segment (start 95.0468 75.311) (end 83.0272 75.311) (width 1.5) (layer "F.Cu") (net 10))
 (segment (start 97.8154 85.2678) (end 97.8154 78.0796) (width 1.5) (layer "F.Cu") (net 10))
 (segment (start 97.8154 78.0796) (end 95.0468 75.311) (width 1.5) (layer "F.Cu") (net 10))
 (segment (start 96.647 90.3986) (end 96.647 88.5444) (width 1.5) (layer "B.Cu") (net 10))
 (segment (start 96.647 88.5444) (end 97.8154 87.376) (width 1.5) (layer "B.Cu") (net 10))
 (segment (start 97.8154 87.376) (end 97.8154 85.2678) (width 1.5) (layer "B.Cu") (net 10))
 (segment (start 95.2754 85.2678) (end 95.2754 87.122) (width 1.5) (layer "F.Cu") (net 2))
 (segment (start 95.2754 82.4992) (end 92.9894 80.2132) (width 1.5) (layer "F.Cu") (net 2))
 (segment (start 99.187 88.8492) (end 99.187 90.3986) (width 1.5) (layer "F.Cu") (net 2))
 (segment (start 95.8342 87.6808) (end 98.0186 87.6808) (width 1.5) (layer "F.Cu") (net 2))
 (segment (start 95.2754 87.122) (end 95.8342 87.6808) (width 1.5) (layer "F.Cu") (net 2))
 (segment (start 92.9894 80.2132) (end 83.2812 80.2132) (width 1.5) (layer "F.Cu") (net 2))
 (segment (start 98.0186 87.6808) (end 99.187 88.8492) (width 1.5) (layer "F.Cu") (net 2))
 (segment (start 95.2754 85.2678) (end 95.2754 82.4992) (width 1.5) (layer "F.Cu") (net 2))
 (segment (start 125.7554 84.8868) (end 125.8062 84.836) (width 1.5) (layer "F.Cu") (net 33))
 (segment (start 119.7864 72.009) (end 125.8062 78.0288) (width 1.5) (layer "F.Cu") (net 33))
 (segment (start 115.57 72.009) (end 114.422 70.861) (width 1) (layer "F.Cu") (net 33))
 (segment (start 115.57 72.009) (end 119.7864 72.009) (width 1.5) (layer "F.Cu") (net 33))
 (segment (start 114.422 70.861) (end 114.422 67.8986) (width 1) (layer "F.Cu") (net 33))
 (segment (start 125.8062 84.836) (end 125.8062 78.0288) (width 1) (layer "F.Cu") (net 33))
 (segment (start 113.538 74.93) (end 112.6744 74.0664) (width 1.5) (layer "F.Cu") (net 32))
 (segment (start 117.5258 74.93) (end 113.538 74.93) (width 1.5) (layer "F.Cu") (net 32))
 (segment (start 111.6076 68.173) (end 111.882 67.8986) (width 1) (layer "F.Cu") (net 32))
 (segment (start 112.6744 74.0664) (end 111.6076 72.9996) (width 1) (layer "F.Cu") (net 32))
 (segment (start 123.2154 80.6196) (end 117.5258 74.93) (width 1.5) (layer "F.Cu") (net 32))
 (segment (start 111.6076 72.9996) (end 111.6076 68.173) (width 1) (layer "F.Cu") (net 32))
 (segment (start 123.2154 84.8868) (end 123.2154 80.6196) (width 1) (layer "F.Cu") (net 32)))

